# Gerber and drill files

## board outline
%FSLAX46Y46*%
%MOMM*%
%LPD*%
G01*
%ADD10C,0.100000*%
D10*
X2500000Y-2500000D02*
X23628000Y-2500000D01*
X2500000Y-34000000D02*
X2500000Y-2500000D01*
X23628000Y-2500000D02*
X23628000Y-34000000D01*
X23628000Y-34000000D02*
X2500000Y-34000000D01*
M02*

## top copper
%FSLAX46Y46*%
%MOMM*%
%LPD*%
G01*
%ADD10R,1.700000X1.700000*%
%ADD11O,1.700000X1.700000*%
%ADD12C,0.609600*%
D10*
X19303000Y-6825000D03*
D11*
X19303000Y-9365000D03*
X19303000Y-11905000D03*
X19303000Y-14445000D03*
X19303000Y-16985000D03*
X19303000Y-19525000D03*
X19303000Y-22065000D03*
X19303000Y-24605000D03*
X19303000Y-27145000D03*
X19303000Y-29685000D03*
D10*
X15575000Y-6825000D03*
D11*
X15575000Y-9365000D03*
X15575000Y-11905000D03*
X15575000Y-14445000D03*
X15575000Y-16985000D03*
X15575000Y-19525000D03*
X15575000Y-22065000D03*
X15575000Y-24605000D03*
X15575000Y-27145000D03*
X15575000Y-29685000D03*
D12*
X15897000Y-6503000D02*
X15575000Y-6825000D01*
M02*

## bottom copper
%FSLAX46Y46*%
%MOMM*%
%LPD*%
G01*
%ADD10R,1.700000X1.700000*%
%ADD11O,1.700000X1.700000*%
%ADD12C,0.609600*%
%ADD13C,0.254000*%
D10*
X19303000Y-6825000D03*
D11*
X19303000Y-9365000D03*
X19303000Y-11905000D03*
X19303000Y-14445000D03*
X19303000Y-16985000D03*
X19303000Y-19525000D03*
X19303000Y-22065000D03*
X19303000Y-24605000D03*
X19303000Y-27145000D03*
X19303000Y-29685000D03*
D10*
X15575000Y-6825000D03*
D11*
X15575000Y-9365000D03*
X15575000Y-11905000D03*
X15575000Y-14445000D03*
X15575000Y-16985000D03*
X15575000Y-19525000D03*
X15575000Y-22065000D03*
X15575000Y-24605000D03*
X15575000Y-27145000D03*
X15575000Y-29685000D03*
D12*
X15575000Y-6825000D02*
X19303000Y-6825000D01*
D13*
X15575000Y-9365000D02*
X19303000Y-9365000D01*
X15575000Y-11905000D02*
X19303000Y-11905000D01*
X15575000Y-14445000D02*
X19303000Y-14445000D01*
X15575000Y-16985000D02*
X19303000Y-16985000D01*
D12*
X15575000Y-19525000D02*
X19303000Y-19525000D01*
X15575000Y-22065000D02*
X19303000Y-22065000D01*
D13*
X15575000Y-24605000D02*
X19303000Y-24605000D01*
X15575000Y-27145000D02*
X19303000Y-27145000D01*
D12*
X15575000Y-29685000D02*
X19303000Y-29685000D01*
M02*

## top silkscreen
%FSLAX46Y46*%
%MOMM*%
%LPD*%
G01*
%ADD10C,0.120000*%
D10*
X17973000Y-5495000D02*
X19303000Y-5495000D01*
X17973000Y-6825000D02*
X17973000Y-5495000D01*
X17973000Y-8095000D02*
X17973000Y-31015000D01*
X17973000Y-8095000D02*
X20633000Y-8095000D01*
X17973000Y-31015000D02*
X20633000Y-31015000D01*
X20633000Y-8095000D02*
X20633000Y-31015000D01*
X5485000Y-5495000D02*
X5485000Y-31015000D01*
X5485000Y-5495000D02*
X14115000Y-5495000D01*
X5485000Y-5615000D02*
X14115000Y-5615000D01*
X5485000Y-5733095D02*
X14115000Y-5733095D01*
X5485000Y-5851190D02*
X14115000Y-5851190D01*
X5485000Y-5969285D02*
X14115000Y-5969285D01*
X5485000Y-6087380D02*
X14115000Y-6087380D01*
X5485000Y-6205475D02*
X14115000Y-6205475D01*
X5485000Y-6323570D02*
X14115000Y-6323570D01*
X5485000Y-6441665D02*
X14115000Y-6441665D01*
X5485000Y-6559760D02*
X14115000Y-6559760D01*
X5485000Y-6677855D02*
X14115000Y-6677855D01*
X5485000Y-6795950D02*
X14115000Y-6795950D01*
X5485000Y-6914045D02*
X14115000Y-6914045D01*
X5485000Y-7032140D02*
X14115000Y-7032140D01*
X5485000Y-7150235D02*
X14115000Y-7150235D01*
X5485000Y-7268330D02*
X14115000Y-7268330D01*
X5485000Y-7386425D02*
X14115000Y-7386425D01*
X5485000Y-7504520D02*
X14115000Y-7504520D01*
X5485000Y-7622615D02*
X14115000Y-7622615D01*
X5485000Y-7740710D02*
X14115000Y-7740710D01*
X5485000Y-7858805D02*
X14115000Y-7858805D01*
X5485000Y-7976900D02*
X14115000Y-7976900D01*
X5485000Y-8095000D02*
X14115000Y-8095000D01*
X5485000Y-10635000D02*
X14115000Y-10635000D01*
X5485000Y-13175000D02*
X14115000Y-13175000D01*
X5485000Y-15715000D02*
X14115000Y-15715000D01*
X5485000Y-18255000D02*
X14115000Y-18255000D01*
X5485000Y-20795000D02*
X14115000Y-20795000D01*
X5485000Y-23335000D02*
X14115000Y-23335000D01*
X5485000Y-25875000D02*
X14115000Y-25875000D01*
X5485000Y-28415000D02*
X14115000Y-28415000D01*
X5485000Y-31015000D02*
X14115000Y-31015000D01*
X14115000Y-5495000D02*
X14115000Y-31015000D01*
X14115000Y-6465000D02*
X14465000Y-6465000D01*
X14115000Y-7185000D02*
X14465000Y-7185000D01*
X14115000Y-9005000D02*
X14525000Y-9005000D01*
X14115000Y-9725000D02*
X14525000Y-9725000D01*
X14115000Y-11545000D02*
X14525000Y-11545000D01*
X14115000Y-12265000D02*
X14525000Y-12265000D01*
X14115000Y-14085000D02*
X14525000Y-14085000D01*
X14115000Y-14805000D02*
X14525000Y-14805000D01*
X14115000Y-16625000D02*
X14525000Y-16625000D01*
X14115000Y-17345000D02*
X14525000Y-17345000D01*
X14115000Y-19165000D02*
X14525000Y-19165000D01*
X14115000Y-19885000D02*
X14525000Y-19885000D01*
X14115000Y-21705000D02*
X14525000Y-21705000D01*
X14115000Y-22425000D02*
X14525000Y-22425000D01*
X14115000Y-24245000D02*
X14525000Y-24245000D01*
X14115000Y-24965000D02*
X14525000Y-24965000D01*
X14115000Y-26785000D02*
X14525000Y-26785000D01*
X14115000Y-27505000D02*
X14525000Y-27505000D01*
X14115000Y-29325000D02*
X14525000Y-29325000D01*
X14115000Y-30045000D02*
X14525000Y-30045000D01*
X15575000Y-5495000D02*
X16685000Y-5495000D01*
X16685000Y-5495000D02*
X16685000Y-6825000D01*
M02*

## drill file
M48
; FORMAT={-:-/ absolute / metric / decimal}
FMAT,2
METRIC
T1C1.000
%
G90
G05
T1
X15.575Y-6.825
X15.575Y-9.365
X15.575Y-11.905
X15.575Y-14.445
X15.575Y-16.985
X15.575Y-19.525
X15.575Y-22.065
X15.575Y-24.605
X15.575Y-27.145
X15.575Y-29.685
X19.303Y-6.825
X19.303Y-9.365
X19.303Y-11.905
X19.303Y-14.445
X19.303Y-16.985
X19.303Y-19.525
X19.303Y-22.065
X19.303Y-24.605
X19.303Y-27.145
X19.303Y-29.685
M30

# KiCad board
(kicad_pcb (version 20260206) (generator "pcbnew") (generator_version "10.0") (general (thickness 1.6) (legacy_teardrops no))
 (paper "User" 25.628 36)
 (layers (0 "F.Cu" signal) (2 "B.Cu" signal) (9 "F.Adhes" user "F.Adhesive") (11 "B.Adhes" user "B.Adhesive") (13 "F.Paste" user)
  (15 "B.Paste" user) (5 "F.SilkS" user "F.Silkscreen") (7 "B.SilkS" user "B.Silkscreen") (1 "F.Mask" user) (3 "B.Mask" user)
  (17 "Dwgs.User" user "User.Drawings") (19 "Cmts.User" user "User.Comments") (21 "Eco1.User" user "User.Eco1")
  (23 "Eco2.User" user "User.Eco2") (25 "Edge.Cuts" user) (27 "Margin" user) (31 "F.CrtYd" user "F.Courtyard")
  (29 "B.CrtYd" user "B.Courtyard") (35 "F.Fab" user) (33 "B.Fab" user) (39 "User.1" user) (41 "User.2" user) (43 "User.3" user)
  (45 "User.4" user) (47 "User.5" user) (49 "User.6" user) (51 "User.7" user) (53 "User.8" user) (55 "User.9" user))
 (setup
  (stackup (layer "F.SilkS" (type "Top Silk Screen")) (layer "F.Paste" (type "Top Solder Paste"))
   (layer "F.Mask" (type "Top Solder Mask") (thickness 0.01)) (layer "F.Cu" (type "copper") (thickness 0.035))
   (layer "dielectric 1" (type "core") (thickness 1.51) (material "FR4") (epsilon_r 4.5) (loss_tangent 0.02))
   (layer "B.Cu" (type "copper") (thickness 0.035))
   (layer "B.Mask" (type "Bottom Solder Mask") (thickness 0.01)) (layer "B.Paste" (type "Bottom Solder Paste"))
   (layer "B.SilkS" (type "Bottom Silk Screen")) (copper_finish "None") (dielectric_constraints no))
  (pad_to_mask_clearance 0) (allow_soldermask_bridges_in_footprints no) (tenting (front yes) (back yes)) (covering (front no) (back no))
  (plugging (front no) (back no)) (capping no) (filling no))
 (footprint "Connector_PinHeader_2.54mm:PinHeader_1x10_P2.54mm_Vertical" (layer "F.Cu") (at 19.303 6.825)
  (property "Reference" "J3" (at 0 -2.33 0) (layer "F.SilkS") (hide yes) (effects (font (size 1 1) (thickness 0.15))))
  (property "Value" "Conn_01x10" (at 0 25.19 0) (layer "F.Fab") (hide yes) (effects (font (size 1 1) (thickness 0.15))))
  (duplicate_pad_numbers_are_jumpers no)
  (fp_line (start -1.33 -1.33) (end 0 -1.33) (stroke (width 0.12) (type solid)) (layer "F.SilkS"))
  (fp_line (start -1.33 0) (end -1.33 -1.33) (stroke (width 0.12) (type solid)) (layer "F.SilkS"))
  (fp_line (start -1.33 1.27) (end -1.33 24.19) (stroke (width 0.12) (type solid)) (layer "F.SilkS"))
  (fp_line (start -1.33 1.27) (end 1.33 1.27) (stroke (width 0.12) (type solid)) (layer "F.SilkS"))
  (fp_line (start -1.33 24.19) (end 1.33 24.19) (stroke (width 0.12) (type solid)) (layer "F.SilkS"))
  (fp_line (start 1.33 1.27) (end 1.33 24.19) (stroke (width 0.12) (type solid)) (layer "F.SilkS"))
  (pad "1" thru_hole rect (at 0 0) (size 1.7 1.7) (drill 1) (layers "*.Cu" "*.Mask") (remove_unused_layers no) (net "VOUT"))
  (pad "2" thru_hole oval (at 0 2.54) (size 1.7 1.7) (drill 1) (layers "*.Cu" "*.Mask") (remove_unused_layers no) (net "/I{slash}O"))
  (pad "3" thru_hole oval (at 0 5.08) (size 1.7 1.7) (drill 1) (layers "*.Cu" "*.Mask") (remove_unused_layers no) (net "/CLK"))
  (pad "4" thru_hole oval (at 0 7.62) (size 1.7 1.7) (drill 1) (layers "*.Cu" "*.Mask") (remove_unused_layers no) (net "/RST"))
  (pad "5" thru_hole oval (at 0 10.16) (size 1.7 1.7) (drill 1) (layers "*.Cu" "*.Mask") (remove_unused_layers no) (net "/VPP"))
  (pad "6" thru_hole oval (at 0 12.7) (size 1.7 1.7) (drill 1) (layers "*.Cu" "*.Mask") (remove_unused_layers no) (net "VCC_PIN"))
  (pad "7" thru_hole oval (at 0 15.24) (size 1.7 1.7) (drill 1) (layers "*.Cu" "*.Mask") (remove_unused_layers no) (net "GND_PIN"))
  (pad "8" thru_hole oval (at 0 17.78) (size 1.7 1.7) (drill 1) (layers "*.Cu" "*.Mask") (remove_unused_layers no) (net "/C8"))
  (pad "9" thru_hole oval (at 0 20.32) (size 1.7 1.7) (drill 1) (layers "*.Cu" "*.Mask") (remove_unused_layers no) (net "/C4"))
  (pad "10" thru_hole oval (at 0 22.86) (size 1.7 1.7) (drill 1) (layers "*.Cu" "*.Mask") (remove_unused_layers no) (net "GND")))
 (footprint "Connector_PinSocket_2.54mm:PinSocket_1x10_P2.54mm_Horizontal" (layer "F.Cu") (at 15.575 6.825)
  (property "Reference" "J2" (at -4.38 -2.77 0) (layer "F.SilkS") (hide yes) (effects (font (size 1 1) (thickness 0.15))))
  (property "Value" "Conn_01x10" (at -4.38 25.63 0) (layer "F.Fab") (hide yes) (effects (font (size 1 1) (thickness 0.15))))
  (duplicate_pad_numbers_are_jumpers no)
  (fp_line (start -10.09 -1.33) (end -10.09 24.19) (stroke (width 0.12) (type solid)) (layer "F.SilkS"))
  (fp_line (start -10.09 -1.33) (end -1.46 -1.33) (stroke (width 0.12) (type solid)) (layer "F.SilkS"))
  (fp_line (start -10.09 -1.21) (end -1.46 -1.21) (stroke (width 0.12) (type solid)) (layer "F.SilkS"))
  (fp_line (start -10.09 -1.091905) (end -1.46 -1.091905) (stroke (width 0.12) (type solid)) (layer "F.SilkS"))
  (fp_line (start -10.09 -0.97381) (end -1.46 -0.97381) (stroke (width 0.12) (type solid)) (layer "F.SilkS"))
  (fp_line (start -10.09 -0.855715) (end -1.46 -0.855715) (stroke (width 0.12) (type solid)) (layer "F.SilkS"))
  (fp_line (start -10.09 -0.73762) (end -1.46 -0.73762) (stroke (width 0.12) (type solid)) (layer "F.SilkS"))
  (fp_line (start -10.09 -0.619525) (end -1.46 -0.619525) (stroke (width 0.12) (type solid)) (layer "F.SilkS"))
  (fp_line (start -10.09 -0.50143) (end -1.46 -0.50143) (stroke (width 0.12) (type solid)) (layer "F.SilkS"))
  (fp_line (start -10.09 -0.383335) (end -1.46 -0.383335) (stroke (width 0.12) (type solid)) (layer "F.SilkS"))
  (fp_line (start -10.09 -0.26524) (end -1.46 -0.26524) (stroke (width 0.12) (type solid)) (layer "F.SilkS"))
  (fp_line (start -10.09 -0.147145) (end -1.46 -0.147145) (stroke (width 0.12) (type solid)) (layer "F.SilkS"))
  (fp_line (start -10.09 -0.02905) (end -1.46 -0.02905) (stroke (width 0.12) (type solid)) (layer "F.SilkS"))
  (fp_line (start -10.09 0.089045) (end -1.46 0.089045) (stroke (width 0.12) (type solid)) (layer "F.SilkS"))
  (fp_line (start -10.09 0.20714) (end -1.46 0.20714) (stroke (width 0.12) (type solid)) (layer "F.SilkS"))
  (fp_line (start -10.09 0.325235) (end -1.46 0.325235) (stroke (width 0.12) (type solid)) (layer "F.SilkS"))
  (fp_line (start -10.09 0.44333) (end -1.46 0.44333) (stroke (width 0.12) (type solid)) (layer "F.SilkS"))
  (fp_line (start -10.09 0.561425) (end -1.46 0.561425) (stroke (width 0.12) (type solid)) (layer "F.SilkS"))
  (fp_line (start -10.09 0.67952) (end -1.46 0.67952) (stroke (width 0.12) (type solid)) (layer "F.SilkS"))
  (fp_line (start -10.09 0.797615) (end -1.46 0.797615) (stroke (width 0.12) (type solid)) (layer "F.SilkS"))
  (fp_line (start -10.09 0.91571) (end -1.46 0.91571) (stroke (width 0.12) (type solid)) (layer "F.SilkS"))
  (fp_line (start -10.09 1.033805) (end -1.46 1.033805) (stroke (width 0.12) (type solid)) (layer "F.SilkS"))
  (fp_line (start -10.09 1.1519) (end -1.46 1.1519) (stroke (width 0.12) (type solid)) (layer "F.SilkS"))
  (fp_line (start -10.09 1.27) (end -1.46 1.27) (stroke (width 0.12) (type solid)) (layer "F.SilkS"))
  (fp_line (start -10.09 3.81) (end -1.46 3.81) (stroke (width 0.12) (type solid)) (layer "F.SilkS"))
  (fp_line (start -10.09 6.35) (end -1.46 6.35) (stroke (width 0.12) (type solid)) (layer "F.SilkS"))
  (fp_line (start -10.09 8.89) (end -1.46 8.89) (stroke (width 0.12) (type solid)) (layer "F.SilkS"))
  (fp_line (start -10.09 11.43) (end -1.46 11.43) (stroke (width 0.12) (type solid)) (layer "F.SilkS"))
  (fp_line (start -10.09 13.97) (end -1.46 13.97) (stroke (width 0.12) (type solid)) (layer "F.SilkS"))
  (fp_line (start -10.09 16.51) (end -1.46 16.51) (stroke (width 0.12) (type solid)) (layer "F.SilkS"))
  (fp_line (start -10.09 19.05) (end -1.46 19.05) (stroke (width 0.12) (type solid)) (layer "F.SilkS"))
  (fp_line (start -10.09 21.59) (end -1.46 21.59) (stroke (width 0.12) (type solid)) (layer "F.SilkS"))
  (fp_line (start -10.09 24.19) (end -1.46 24.19) (stroke (width 0.12) (type solid)) (layer "F.SilkS"))
  (fp_line (start -1.46 -1.33) (end -1.46 24.19) (stroke (width 0.12) (type solid)) (layer "F.SilkS"))
  (fp_line (start -1.46 -0.36) (end -1.11 -0.36) (stroke (width 0.12) (type solid)) (layer "F.SilkS"))
  (fp_line (start -1.46 0.36) (end -1.11 0.36) (stroke (width 0.12) (type solid)) (layer "F.SilkS"))
  (fp_line (start -1.46 2.18) (end -1.05 2.18) (stroke (width 0.12) (type solid)) (layer "F.SilkS"))
  (fp_line (start -1.46 2.9) (end -1.05 2.9) (stroke (width 0.12) (type solid)) (layer "F.SilkS"))
  (fp_line (start -1.46 4.72) (end -1.05 4.72) (stroke (width 0.12) (type solid)) (layer "F.SilkS"))
  (fp_line (start -1.46 5.44) (end -1.05 5.44) (stroke (width 0.12) (type solid)) (layer "F.SilkS"))
  (fp_line (start -1.46 7.26) (end -1.05 7.26) (stroke (width 0.12) (type solid)) (layer "F.SilkS"))
  (fp_line (start -1.46 7.98) (end -1.05 7.98) (stroke (width 0.12) (type solid)) (layer "F.SilkS"))
  (fp_line (start -1.46 9.8) (end -1.05 9.8) (stroke (width 0.12) (type solid)) (layer "F.SilkS"))
  (fp_line (start -1.46 10.52) (end -1.05 10.52) (stroke (width 0.12) (type solid)) (layer "F.SilkS"))
  (fp_line (start -1.46 12.34) (end -1.05 12.34) (stroke (width 0.12) (type solid)) (layer "F.SilkS"))
  (fp_line (start -1.46 13.06) (end -1.05 13.06) (stroke (width 0.12) (type solid)) (layer "F.SilkS"))
  (fp_line (start -1.46 14.88) (end -1.05 14.88) (stroke (width 0.12) (type solid)) (layer "F.SilkS"))
  (fp_line (start -1.46 15.6) (end -1.05 15.6) (stroke (width 0.12) (type solid)) (layer "F.SilkS"))
  (fp_line (start -1.46 17.42) (end -1.05 17.42) (stroke (width 0.12) (type solid)) (layer "F.SilkS"))
  (fp_line (start -1.46 18.14) (end -1.05 18.14) (stroke (width 0.12) (type solid)) (layer "F.SilkS"))
  (fp_line (start -1.46 19.96) (end -1.05 19.96) (stroke (width 0.12) (type solid)) (layer "F.SilkS"))
  (fp_line (start -1.46 20.68) (end -1.05 20.68) (stroke (width 0.12) (type solid)) (layer "F.SilkS"))
  (fp_line (start -1.46 22.5) (end -1.05 22.5) (stroke (width 0.12) (type solid)) (layer "F.SilkS"))
  (fp_line (start -1.46 23.22) (end -1.05 23.22) (stroke (width 0.12) (type solid)) (layer "F.SilkS"))
  (fp_line (start 0 -1.33) (end 1.11 -1.33) (stroke (width 0.12) (type solid)) (layer "F.SilkS"))
  (fp_line (start 1.11 -1.33) (end 1.11 0) (stroke (width 0.12) (type solid)) (layer "F.SilkS"))
  (pad "1" thru_hole rect (at 0 0) (size 1.7 1.7) (drill 1) (layers "*.Cu" "*.Mask") (remove_unused_layers no) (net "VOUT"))
  (pad "2" thru_hole oval (at 0 2.54) (size 1.7 1.7) (drill 1) (layers "*.Cu" "*.Mask") (remove_unused_layers no) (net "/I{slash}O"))
  (pad "3" thru_hole oval (at 0 5.08) (size 1.7 1.7) (drill 1) (layers "*.Cu" "*.Mask") (remove_unused_layers no) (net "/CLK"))
  (pad "4" thru_hole oval (at 0 7.62) (size 1.7 1.7) (drill 1) (layers "*.Cu" "*.Mask") (remove_unused_layers no) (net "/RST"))
  (pad "5" thru_hole oval (at 0 10.16) (size 1.7 1.7) (drill 1) (layers "*.Cu" "*.Mask") (remove_unused_layers no) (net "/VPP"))
  (pad "6" thru_hole oval (at 0 12.7) (size 1.7 1.7) (drill 1) (layers "*.Cu" "*.Mask") (remove_unused_layers no) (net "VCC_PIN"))
  (pad "7" thru_hole oval (at 0 15.24) (size 1.7 1.7) (drill 1) (layers "*.Cu" "*.Mask") (remove_unused_layers no) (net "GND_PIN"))
  (pad "8" thru_hole oval (at 0 17.78) (size 1.7 1.7) (drill 1) (layers "*.Cu" "*.Mask") (remove_unused_layers no) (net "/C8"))
  (pad "9" thru_hole oval (at 0 20.32) (size 1.7 1.7) (drill 1) (layers "*.Cu" "*.Mask") (remove_unused_layers no) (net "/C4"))
  (pad "10" thru_hole oval (at 0 22.86) (size 1.7 1.7) (drill 1) (layers "*.Cu" "*.Mask") (remove_unused_layers no) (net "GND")))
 (gr_line (start 2.5 2.5) (end 23.628 2.5) (stroke (width 0.1) (type default)) (layer "Edge.Cuts"))
 (gr_line (start 2.5 34) (end 2.5 2.5) (stroke (width 0.1) (type default)) (layer "Edge.Cuts"))
 (gr_line (start 23.628 2.5) (end 23.628 34) (stroke (width 0.1) (type default)) (layer "Edge.Cuts"))
 (gr_line (start 23.628 34) (end 2.5 34) (stroke (width 0.1) (type default)) (layer "Edge.Cuts"))
 (segment (start 15.897 6.503) (end 15.575 6.825) (width 0.6096) (layer "F.Cu") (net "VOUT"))
 (segment (start 15.575 6.825) (end 19.303 6.825) (width 0.6096) (layer "B.Cu") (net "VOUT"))
 (segment (start 15.575 9.365) (end 19.303 9.365) (width 0.254) (layer "B.Cu") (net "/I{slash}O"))
 (segment (start 15.575 11.905) (end 19.303 11.905) (width 0.254) (layer "B.Cu") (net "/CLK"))
 (segment (start 15.575 14.445) (end 19.303 14.445) (width 0.254) (layer "B.Cu") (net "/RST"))
 (segment (start 15.575 16.985) (end 19.303 16.985) (width 0.254) (layer "B.Cu") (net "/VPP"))
 (segment (start 15.575 19.525) (end 19.303 19.525) (width 0.6096) (layer "B.Cu") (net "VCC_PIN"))
 (segment (start 15.575 22.065) (end 19.303 22.065) (width 0.6096) (layer "B.Cu") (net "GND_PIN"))
 (segment (start 15.575 24.605) (end 19.303 24.605) (width 0.254) (layer "B.Cu") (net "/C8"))
 (segment (start 15.575 27.145) (end 19.303 27.145) (width 0.254) (layer "B.Cu") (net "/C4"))
 (segment (start 15.575 29.685) (end 19.303 29.685) (width 0.6096) (layer "B.Cu") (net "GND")))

